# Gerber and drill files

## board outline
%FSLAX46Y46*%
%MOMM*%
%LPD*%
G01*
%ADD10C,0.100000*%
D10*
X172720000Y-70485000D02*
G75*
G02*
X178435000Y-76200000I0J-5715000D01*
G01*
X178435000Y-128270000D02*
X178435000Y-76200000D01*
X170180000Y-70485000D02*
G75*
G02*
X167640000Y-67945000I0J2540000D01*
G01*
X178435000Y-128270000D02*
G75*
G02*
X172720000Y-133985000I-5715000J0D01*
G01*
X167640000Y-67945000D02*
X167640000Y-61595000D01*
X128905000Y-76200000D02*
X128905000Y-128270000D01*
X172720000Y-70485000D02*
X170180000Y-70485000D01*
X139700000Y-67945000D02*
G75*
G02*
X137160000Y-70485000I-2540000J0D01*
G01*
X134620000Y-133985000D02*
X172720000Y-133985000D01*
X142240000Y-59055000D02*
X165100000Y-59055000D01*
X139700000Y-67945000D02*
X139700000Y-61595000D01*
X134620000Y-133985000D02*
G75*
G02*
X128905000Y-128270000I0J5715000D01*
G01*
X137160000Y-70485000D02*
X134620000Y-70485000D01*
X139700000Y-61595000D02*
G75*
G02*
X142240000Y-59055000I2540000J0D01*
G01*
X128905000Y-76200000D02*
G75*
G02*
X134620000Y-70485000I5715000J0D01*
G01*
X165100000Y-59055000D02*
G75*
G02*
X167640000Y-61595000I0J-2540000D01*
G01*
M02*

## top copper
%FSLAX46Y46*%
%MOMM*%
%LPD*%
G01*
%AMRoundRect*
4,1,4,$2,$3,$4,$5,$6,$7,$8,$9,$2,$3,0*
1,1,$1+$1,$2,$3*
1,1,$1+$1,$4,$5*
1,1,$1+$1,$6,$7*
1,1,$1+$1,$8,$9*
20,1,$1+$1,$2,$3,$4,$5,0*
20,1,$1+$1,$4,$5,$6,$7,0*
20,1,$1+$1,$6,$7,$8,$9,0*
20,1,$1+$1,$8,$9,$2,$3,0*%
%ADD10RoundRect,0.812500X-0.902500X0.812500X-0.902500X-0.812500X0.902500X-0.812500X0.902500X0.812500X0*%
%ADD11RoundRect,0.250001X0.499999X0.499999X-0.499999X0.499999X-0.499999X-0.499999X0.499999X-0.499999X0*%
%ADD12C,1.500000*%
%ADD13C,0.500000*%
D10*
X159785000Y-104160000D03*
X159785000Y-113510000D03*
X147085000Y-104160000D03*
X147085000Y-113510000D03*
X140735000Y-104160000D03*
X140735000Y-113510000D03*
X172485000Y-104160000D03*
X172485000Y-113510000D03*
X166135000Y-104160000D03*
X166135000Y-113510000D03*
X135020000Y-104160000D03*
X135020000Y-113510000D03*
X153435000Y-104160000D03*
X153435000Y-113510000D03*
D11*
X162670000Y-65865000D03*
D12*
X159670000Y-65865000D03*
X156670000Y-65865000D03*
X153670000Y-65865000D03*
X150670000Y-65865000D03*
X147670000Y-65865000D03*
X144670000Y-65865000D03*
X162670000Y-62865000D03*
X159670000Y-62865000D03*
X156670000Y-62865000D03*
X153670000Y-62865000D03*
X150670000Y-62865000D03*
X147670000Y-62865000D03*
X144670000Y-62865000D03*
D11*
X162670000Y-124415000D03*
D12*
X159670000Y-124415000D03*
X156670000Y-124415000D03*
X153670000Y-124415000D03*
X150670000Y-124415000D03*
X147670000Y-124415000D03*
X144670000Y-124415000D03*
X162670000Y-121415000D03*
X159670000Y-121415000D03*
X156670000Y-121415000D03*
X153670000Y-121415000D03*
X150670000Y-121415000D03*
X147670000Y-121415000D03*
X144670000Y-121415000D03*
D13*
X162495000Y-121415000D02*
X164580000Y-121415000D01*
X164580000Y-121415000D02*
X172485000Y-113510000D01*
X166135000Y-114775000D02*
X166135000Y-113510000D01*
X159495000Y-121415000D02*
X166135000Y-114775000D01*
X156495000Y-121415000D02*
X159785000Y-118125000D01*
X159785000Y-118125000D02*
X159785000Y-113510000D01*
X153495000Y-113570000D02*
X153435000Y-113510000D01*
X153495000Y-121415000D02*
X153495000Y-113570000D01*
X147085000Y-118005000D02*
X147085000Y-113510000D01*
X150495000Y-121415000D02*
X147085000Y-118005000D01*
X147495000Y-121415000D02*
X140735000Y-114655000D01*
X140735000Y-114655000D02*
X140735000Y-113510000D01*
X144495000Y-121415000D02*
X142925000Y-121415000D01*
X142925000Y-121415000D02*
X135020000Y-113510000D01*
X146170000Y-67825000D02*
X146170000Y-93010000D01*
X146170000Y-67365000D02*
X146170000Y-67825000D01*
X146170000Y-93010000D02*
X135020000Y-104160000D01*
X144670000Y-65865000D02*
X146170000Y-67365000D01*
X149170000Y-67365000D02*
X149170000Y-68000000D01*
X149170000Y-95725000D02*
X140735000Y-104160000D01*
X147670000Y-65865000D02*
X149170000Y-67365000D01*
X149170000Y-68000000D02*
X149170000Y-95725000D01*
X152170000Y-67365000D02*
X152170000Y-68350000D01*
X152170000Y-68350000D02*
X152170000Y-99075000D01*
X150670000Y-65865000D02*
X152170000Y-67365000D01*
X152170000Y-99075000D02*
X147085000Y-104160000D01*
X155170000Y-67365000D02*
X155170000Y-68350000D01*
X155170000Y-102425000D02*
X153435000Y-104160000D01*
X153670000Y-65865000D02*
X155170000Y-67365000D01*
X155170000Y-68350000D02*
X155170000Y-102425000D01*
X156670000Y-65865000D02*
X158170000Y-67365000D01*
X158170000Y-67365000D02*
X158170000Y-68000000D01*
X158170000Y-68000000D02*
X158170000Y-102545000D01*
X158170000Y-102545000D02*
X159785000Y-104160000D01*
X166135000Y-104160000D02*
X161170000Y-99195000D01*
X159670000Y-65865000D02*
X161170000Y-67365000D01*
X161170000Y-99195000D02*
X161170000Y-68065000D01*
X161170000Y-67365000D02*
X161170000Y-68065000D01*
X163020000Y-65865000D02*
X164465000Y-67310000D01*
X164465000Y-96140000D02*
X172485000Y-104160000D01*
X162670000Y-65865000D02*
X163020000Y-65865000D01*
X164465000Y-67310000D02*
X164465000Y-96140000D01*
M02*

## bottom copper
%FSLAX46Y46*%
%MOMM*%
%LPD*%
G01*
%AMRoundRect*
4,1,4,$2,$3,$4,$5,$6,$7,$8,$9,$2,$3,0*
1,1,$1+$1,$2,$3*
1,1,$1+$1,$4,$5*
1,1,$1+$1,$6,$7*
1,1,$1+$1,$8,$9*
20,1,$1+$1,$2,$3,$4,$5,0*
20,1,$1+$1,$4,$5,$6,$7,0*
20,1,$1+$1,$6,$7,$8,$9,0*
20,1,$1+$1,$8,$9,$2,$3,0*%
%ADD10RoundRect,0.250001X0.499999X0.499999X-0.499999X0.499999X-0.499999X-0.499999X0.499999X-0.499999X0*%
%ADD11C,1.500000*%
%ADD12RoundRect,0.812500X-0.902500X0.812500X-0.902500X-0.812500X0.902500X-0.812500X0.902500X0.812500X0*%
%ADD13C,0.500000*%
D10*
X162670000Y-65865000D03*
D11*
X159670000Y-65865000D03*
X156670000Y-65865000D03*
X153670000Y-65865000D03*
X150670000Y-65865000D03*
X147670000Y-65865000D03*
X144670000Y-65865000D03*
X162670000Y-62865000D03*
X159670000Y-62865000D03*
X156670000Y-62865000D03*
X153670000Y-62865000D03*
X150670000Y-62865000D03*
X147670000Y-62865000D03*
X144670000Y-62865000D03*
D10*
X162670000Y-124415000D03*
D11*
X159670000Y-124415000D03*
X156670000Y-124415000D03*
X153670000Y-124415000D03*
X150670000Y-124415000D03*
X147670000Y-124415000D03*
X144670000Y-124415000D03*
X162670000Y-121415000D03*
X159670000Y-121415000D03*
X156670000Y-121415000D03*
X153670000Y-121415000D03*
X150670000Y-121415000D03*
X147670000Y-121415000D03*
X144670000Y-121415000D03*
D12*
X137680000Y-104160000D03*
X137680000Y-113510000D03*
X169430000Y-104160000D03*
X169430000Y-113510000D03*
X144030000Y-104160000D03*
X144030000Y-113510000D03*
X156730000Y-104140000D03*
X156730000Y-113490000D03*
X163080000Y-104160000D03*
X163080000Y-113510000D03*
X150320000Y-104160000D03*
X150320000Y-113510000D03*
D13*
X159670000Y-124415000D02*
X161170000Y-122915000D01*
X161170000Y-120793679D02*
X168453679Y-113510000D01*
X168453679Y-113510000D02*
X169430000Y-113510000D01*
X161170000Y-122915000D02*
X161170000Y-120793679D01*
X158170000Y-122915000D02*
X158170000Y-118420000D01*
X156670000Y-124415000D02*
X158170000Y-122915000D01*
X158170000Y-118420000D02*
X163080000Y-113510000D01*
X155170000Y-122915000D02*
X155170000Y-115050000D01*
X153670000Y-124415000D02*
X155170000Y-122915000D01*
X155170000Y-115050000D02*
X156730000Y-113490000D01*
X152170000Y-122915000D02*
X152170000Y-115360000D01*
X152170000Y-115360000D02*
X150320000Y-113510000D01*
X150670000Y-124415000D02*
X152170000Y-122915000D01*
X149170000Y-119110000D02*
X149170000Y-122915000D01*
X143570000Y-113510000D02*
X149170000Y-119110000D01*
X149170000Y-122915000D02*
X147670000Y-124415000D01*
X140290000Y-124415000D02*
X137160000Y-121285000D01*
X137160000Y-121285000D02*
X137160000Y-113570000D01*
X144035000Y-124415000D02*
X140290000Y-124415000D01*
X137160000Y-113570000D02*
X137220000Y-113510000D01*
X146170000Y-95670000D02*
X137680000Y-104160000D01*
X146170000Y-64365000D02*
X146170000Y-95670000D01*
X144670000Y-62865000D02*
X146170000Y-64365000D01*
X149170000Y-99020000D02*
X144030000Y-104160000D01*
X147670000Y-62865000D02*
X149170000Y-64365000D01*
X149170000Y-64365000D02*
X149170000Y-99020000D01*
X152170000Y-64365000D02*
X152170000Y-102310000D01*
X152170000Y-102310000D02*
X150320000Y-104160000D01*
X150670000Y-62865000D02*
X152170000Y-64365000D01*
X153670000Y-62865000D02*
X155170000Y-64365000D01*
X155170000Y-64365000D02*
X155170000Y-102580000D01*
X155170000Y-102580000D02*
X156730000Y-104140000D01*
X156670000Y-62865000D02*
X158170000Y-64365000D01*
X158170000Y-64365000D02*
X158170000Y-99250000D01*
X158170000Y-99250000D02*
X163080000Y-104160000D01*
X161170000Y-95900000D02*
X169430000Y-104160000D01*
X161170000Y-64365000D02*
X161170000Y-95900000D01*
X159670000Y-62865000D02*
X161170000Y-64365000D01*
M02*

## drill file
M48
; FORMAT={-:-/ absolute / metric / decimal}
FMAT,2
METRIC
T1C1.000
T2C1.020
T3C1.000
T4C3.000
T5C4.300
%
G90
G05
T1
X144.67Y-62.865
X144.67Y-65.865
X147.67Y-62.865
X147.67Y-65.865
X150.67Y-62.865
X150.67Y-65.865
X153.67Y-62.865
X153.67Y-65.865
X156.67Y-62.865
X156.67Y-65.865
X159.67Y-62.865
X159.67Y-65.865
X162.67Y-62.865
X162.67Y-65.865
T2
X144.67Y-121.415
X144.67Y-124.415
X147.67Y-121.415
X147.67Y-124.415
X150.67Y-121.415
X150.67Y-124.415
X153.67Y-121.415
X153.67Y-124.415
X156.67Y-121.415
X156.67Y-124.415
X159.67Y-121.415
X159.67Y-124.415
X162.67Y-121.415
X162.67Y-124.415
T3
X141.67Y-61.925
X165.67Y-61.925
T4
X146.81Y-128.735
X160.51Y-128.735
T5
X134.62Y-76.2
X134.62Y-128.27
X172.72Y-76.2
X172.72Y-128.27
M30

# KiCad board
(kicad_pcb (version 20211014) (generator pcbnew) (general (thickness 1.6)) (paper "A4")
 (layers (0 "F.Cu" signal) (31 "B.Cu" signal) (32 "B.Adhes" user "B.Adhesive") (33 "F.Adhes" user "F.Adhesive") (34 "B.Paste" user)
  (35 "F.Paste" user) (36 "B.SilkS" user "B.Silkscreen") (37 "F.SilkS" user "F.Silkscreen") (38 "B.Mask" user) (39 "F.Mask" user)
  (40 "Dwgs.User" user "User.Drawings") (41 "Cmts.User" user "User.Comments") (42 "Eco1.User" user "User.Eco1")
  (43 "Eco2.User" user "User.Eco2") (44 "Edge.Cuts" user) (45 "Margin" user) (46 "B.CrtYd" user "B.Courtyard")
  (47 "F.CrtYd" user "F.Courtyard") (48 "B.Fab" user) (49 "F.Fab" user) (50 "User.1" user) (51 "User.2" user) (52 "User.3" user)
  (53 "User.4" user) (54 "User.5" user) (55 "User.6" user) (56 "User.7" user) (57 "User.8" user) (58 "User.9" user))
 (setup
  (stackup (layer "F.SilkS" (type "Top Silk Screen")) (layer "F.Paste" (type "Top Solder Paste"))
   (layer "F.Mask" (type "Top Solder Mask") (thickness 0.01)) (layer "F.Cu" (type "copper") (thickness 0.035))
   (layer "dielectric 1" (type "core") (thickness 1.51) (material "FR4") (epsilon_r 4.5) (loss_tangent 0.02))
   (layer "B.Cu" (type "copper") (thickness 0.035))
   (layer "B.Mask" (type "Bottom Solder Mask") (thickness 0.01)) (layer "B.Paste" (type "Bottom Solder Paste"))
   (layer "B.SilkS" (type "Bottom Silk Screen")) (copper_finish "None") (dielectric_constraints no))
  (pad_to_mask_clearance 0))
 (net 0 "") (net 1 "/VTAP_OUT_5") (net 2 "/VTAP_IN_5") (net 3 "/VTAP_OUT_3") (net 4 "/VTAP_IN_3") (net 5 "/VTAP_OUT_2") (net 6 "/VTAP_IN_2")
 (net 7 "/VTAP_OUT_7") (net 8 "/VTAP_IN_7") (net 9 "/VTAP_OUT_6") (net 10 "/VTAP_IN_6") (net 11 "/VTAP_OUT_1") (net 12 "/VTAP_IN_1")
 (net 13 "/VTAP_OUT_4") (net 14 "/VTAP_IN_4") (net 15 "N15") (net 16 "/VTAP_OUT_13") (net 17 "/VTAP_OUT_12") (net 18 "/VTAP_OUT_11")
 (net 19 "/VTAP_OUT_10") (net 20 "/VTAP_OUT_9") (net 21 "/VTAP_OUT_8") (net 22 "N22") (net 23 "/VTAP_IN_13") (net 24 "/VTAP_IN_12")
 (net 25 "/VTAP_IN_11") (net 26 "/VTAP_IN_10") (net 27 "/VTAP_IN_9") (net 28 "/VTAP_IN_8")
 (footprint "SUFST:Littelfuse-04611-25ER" (layer "F.Cu") (at 159.845 108.585 -90)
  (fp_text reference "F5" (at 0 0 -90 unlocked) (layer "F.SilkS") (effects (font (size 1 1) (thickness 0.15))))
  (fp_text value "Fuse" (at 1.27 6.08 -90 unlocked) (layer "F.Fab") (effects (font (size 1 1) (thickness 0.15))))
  (pad "1" smd roundrect (at -4.425 0.06 270) (size 3.25 3.43) (layers "F.Cu" "F.Paste" "F.Mask") (roundrect_rratio 0.25)
   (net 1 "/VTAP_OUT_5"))
  (pad "2" smd roundrect (at 4.925 0.06 270) (size 3.25 3.43) (layers "F.Cu" "F.Paste" "F.Mask") (roundrect_rratio 0.25)
   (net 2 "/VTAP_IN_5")))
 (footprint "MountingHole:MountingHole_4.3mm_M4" (layer "F.Cu") (at 172.72 76.2)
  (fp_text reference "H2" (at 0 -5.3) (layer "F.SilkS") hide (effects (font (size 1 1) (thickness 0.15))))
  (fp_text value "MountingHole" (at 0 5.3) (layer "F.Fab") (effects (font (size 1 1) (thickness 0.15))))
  (pad "" np_thru_hole circle (at 0 0) (size 4.3 4.3) (drill 4.3) (layers *.Cu *.Mask)))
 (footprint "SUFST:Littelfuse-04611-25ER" (layer "F.Cu") (at 147.145 108.585 -90)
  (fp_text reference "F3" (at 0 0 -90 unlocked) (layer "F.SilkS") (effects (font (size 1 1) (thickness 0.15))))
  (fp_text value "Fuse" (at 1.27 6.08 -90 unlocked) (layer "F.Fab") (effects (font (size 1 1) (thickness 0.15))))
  (pad "1" smd roundrect (at -4.425 0.06 270) (size 3.25 3.43) (layers "F.Cu" "F.Paste" "F.Mask") (roundrect_rratio 0.25)
   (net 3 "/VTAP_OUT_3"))
  (pad "2" smd roundrect (at 4.925 0.06 270) (size 3.25 3.43) (layers "F.Cu" "F.Paste" "F.Mask") (roundrect_rratio 0.25)
   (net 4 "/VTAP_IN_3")))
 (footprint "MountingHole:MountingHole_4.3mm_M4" (layer "F.Cu") (at 172.72 128.27)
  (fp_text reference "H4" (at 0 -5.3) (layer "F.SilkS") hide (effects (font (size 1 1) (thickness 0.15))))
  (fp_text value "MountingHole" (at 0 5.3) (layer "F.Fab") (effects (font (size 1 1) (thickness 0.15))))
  (pad "" np_thru_hole circle (at 0 0) (size 4.3 4.3) (drill 4.3) (layers *.Cu *.Mask)))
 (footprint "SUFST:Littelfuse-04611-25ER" (layer "F.Cu") (at 140.795 108.585 -90)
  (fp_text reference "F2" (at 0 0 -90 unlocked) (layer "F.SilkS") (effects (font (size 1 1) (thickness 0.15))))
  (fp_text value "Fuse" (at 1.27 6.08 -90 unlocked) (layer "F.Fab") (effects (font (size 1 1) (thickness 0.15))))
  (pad "1" smd roundrect (at -4.425 0.06 270) (size 3.25 3.43) (layers "F.Cu" "F.Paste" "F.Mask") (roundrect_rratio 0.25)
   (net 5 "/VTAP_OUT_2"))
  (pad "2" smd roundrect (at 4.925 0.06 270) (size 3.25 3.43) (layers "F.Cu" "F.Paste" "F.Mask") (roundrect_rratio 0.25)
   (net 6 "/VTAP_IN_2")))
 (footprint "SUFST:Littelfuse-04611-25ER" (layer "F.Cu") (at 172.545 108.585 -90)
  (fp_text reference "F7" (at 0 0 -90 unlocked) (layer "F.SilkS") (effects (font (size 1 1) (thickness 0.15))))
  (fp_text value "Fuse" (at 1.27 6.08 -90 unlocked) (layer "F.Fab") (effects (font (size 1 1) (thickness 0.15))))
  (pad "1" smd roundrect (at -4.425 0.06 270) (size 3.25 3.43) (layers "F.Cu" "F.Paste" "F.Mask") (roundrect_rratio 0.25)
   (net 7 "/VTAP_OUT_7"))
  (pad "2" smd roundrect (at 4.925 0.06 270) (size 3.25 3.43) (layers "F.Cu" "F.Paste" "F.Mask") (roundrect_rratio 0.25)
   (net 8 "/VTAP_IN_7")))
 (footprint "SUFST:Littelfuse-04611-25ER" (layer "F.Cu") (at 166.195 108.585 -90)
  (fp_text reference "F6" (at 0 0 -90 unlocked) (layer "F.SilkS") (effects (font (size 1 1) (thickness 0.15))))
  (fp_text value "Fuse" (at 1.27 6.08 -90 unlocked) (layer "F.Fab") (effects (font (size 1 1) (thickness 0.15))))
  (pad "1" smd roundrect (at -4.425 0.06 270) (size 3.25 3.43) (layers "F.Cu" "F.Paste" "F.Mask") (roundrect_rratio 0.25)
   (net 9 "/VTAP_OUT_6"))
  (pad "2" smd roundrect (at 4.925 0.06 270) (size 3.25 3.43) (layers "F.Cu" "F.Paste" "F.Mask") (roundrect_rratio 0.25)
   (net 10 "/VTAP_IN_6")))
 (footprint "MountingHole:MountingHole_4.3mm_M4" (layer "F.Cu") (at 134.62 128.27)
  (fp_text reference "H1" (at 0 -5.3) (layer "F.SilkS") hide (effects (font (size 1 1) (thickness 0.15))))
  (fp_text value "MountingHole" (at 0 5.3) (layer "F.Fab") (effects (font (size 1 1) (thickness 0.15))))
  (pad "" np_thru_hole circle (at 0 0) (size 4.3 4.3) (drill 4.3) (layers *.Cu *.Mask)))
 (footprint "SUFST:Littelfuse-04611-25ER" (layer "F.Cu") (at 135.08 108.585 -90)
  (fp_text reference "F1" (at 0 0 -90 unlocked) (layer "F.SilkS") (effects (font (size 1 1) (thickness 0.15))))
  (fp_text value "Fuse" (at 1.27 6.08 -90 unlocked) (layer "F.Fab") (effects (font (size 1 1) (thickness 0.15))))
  (pad "1" smd roundrect (at -4.425 0.06 270) (size 3.25 3.43) (layers "F.Cu" "F.Paste" "F.Mask") (roundrect_rratio 0.25)
   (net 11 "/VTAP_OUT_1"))
  (pad "2" smd roundrect (at 4.925 0.06 270) (size 3.25 3.43) (layers "F.Cu" "F.Paste" "F.Mask") (roundrect_rratio 0.25)
   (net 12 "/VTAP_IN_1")))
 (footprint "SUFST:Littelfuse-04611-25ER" (layer "F.Cu") (at 153.495 108.585 -90)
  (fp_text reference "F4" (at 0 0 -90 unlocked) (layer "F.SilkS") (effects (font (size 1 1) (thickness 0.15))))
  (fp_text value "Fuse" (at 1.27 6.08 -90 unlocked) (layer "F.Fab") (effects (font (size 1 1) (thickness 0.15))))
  (pad "1" smd roundrect (at -4.425 0.06 270) (size 3.25 3.43) (layers "F.Cu" "F.Paste" "F.Mask") (roundrect_rratio 0.25)
   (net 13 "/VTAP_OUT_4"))
  (pad "2" smd roundrect (at 4.925 0.06 270) (size 3.25 3.43) (layers "F.Cu" "F.Paste" "F.Mask") (roundrect_rratio 0.25)
   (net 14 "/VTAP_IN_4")))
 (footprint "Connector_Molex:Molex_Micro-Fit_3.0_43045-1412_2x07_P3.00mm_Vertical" (layer "F.Cu") (at 162.67 65.865 180)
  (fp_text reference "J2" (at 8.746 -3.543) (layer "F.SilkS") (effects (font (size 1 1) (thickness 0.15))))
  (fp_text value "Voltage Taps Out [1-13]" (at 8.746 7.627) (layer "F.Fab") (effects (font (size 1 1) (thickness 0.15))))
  (pad "" np_thru_hole circle (at 21 3.94 180) (size 1 1) (drill 1) (layers *.Cu *.Mask))
  (pad "" np_thru_hole circle (at -3 3.94 180) (size 1 1) (drill 1) (layers *.Cu *.Mask))
  (pad "1" thru_hole roundrect (at 0 0 180) (size 1.5 1.5) (drill 1) (layers *.Cu *.Mask) (roundrect_rratio 0.166667) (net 7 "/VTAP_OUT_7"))
  (pad "2" thru_hole circle (at 3 0 180) (size 1.5 1.5) (drill 1) (layers *.Cu *.Mask) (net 9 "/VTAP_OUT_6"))
  (pad "3" thru_hole circle (at 6 0 180) (size 1.5 1.5) (drill 1) (layers *.Cu *.Mask) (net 1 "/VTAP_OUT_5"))
  (pad "4" thru_hole circle (at 9 0 180) (size 1.5 1.5) (drill 1) (layers *.Cu *.Mask) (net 13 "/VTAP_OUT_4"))
  (pad "5" thru_hole circle (at 12 0 180) (size 1.5 1.5) (drill 1) (layers *.Cu *.Mask) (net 3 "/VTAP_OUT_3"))
  (pad "6" thru_hole circle (at 15 0 180) (size 1.5 1.5) (drill 1) (layers *.Cu *.Mask) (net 5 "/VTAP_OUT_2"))
  (pad "7" thru_hole circle (at 18 0 180) (size 1.5 1.5) (drill 1) (layers *.Cu *.Mask) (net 11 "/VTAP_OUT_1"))
  (pad "8" thru_hole circle (at 0 3 180) (size 1.5 1.5) (drill 1) (layers *.Cu *.Mask) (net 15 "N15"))
  (pad "9" thru_hole circle (at 3 3 180) (size 1.5 1.5) (drill 1) (layers *.Cu *.Mask) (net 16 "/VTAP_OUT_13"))
  (pad "10" thru_hole circle (at 6 3 180) (size 1.5 1.5) (drill 1) (layers *.Cu *.Mask) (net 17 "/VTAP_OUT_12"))
  (pad "11" thru_hole circle (at 9 3 180) (size 1.5 1.5) (drill 1) (layers *.Cu *.Mask) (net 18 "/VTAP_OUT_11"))
  (pad "12" thru_hole circle (at 12 3 180) (size 1.5 1.5) (drill 1) (layers *.Cu *.Mask) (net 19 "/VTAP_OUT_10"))
  (pad "13" thru_hole circle (at 15 3 180) (size 1.5 1.5) (drill 1) (layers *.Cu *.Mask) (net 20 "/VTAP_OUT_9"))
  (pad "14" thru_hole circle (at 18 3 180) (size 1.5 1.5) (drill 1) (layers *.Cu *.Mask) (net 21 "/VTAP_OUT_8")))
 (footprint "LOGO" (layer "F.Cu") (at 153.67 85.09)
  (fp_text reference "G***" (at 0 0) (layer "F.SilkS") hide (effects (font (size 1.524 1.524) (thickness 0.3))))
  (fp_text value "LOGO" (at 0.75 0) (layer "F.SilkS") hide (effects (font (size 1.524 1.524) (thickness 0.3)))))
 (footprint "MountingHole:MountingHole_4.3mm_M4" (layer "F.Cu") (at 134.62 76.2)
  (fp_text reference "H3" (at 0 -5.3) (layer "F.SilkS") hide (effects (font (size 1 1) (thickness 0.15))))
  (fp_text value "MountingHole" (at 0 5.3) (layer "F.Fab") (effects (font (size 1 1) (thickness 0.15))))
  (pad "" np_thru_hole circle (at 0 0) (size 4.3 4.3) (drill 4.3) (layers *.Cu *.Mask)))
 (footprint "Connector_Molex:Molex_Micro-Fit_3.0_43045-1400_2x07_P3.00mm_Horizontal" (layer "F.Cu") (at 162.67 124.415 180)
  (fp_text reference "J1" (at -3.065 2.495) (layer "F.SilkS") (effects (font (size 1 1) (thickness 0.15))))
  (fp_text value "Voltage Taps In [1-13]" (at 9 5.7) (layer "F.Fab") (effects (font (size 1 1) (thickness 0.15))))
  (pad "" np_thru_hole circle (at 15.86 -4.32 180) (size 3 3) (drill 3) (layers *.Cu *.Mask))
  (pad "" np_thru_hole circle (at 2.16 -4.32 180) (size 3 3) (drill 3) (layers *.Cu *.Mask))
  (pad "1" thru_hole roundrect (at 0 0 180) (size 1.5 1.5) (drill 1.02) (layers *.Cu *.Mask) (roundrect_rratio 0.166667) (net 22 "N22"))
  (pad "2" thru_hole circle (at 3 0 180) (size 1.5 1.5) (drill 1.02) (layers *.Cu *.Mask) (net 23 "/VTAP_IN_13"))
  (pad "3" thru_hole circle (at 6 0 180) (size 1.5 1.5) (drill 1.02) (layers *.Cu *.Mask) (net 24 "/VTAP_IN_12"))
  (pad "4" thru_hole circle (at 9 0 180) (size 1.5 1.5) (drill 1.02) (layers *.Cu *.Mask) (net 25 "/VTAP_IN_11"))
  (pad "5" thru_hole circle (at 12 0 180) (size 1.5 1.5) (drill 1.02) (layers *.Cu *.Mask) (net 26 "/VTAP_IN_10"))
  (pad "6" thru_hole circle (at 15 0 180) (size 1.5 1.5) (drill 1.02) (layers *.Cu *.Mask) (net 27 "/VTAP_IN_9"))
  (pad "7" thru_hole circle (at 18 0 180) (size 1.5 1.5) (drill 1.02) (layers *.Cu *.Mask) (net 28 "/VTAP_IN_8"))
  (pad "8" thru_hole circle (at 0 3 180) (size 1.5 1.5) (drill 1.02) (layers *.Cu *.Mask) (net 8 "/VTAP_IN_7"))
  (pad "9" thru_hole circle (at 3 3 180) (size 1.5 1.5) (drill 1.02) (layers *.Cu *.Mask) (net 10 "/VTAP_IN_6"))
  (pad "10" thru_hole circle (at 6 3 180) (size 1.5 1.5) (drill 1.02) (layers *.Cu *.Mask) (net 2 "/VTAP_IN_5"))
  (pad "11" thru_hole circle (at 9 3 180) (size 1.5 1.5) (drill 1.02) (layers *.Cu *.Mask) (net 14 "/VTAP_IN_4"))
  (pad "12" thru_hole circle (at 12 3 180) (size 1.5 1.5) (drill 1.02) (layers *.Cu *.Mask) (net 4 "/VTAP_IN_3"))
  (pad "13" thru_hole circle (at 15 3 180) (size 1.5 1.5) (drill 1.02) (layers *.Cu *.Mask) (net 6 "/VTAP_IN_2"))
  (pad "14" thru_hole circle (at 18 3 180) (size 1.5 1.5) (drill 1.02) (layers *.Cu *.Mask) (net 12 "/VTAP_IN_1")))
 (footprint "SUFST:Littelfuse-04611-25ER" (layer "B.Cu") (at 137.62 108.585 -90)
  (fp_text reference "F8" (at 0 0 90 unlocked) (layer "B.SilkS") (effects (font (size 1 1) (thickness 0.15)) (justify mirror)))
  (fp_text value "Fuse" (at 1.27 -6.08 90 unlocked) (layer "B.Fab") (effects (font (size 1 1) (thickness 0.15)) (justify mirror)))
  (pad "1" smd roundrect (at -4.425 -0.06 270) (size 3.25 3.43) (layers "B.Cu" "B.Paste" "B.Mask") (roundrect_rratio 0.25)
   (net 21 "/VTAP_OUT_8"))
  (pad "2" smd roundrect (at 4.925 -0.06 270) (size 3.25 3.43) (layers "B.Cu" "B.Paste" "B.Mask") (roundrect_rratio 0.25)
   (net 28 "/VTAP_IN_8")))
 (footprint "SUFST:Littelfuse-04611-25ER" (layer "B.Cu") (at 169.37 108.585 -90)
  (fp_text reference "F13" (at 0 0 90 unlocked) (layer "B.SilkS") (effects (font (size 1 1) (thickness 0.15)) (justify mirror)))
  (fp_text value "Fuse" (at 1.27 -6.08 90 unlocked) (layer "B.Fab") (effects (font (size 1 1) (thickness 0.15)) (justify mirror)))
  (pad "1" smd roundrect (at -4.425 -0.06 270) (size 3.25 3.43) (layers "B.Cu" "B.Paste" "B.Mask") (roundrect_rratio 0.25)
   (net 16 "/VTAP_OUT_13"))
  (pad "2" smd roundrect (at 4.925 -0.06 270) (size 3.25 3.43) (layers "B.Cu" "B.Paste" "B.Mask") (roundrect_rratio 0.25)
   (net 23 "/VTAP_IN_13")))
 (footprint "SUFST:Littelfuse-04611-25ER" (layer "B.Cu") (at 143.97 108.585 -90)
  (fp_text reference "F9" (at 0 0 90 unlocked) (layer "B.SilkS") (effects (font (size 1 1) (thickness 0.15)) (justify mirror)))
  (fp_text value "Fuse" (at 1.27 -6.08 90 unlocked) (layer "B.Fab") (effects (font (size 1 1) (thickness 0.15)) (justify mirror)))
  (pad "1" smd roundrect (at -4.425 -0.06 270) (size 3.25 3.43) (layers "B.Cu" "B.Paste" "B.Mask") (roundrect_rratio 0.25)
   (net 20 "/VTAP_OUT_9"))
  (pad "2" smd roundrect (at 4.925 -0.06 270) (size 3.25 3.43) (layers "B.Cu" "B.Paste" "B.Mask") (roundrect_rratio 0.25)
   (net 27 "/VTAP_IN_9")))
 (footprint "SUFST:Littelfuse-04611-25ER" (layer "B.Cu") (at 156.67 108.565 -90)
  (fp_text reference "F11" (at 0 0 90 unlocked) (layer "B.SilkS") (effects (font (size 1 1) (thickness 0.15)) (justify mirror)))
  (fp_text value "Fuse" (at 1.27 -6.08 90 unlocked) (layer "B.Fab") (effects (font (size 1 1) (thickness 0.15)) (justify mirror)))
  (pad "1" smd roundrect (at -4.425 -0.06 270) (size 3.25 3.43) (layers "B.Cu" "B.Paste" "B.Mask") (roundrect_rratio 0.25)
   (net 18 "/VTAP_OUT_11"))
  (pad "2" smd roundrect (at 4.925 -0.06 270) (size 3.25 3.43) (layers "B.Cu" "B.Paste" "B.Mask") (roundrect_rratio 0.25)
   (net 25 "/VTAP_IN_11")))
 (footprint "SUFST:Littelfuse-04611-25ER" (layer "B.Cu") (at 163.02 108.585 -90)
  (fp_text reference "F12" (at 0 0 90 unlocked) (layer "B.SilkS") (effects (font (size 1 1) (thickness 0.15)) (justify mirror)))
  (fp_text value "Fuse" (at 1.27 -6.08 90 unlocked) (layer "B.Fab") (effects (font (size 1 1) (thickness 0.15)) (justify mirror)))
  (pad "1" smd roundrect (at -4.425 -0.06 270) (size 3.25 3.43) (layers "B.Cu" "B.Paste" "B.Mask") (roundrect_rratio 0.25)
   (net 17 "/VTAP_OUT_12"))
  (pad "2" smd roundrect (at 4.925 -0.06 270) (size 3.25 3.43) (layers "B.Cu" "B.Paste" "B.Mask") (roundrect_rratio 0.25)
   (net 24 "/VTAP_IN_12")))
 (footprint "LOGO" (layer "B.Cu") (at 153.67 85.09 180)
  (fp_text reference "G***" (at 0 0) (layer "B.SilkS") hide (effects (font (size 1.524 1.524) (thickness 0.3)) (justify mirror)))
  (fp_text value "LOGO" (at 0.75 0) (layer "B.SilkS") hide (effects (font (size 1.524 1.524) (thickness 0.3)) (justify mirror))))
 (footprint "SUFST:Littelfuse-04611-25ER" (layer "B.Cu") (at 150.26 108.585 -90)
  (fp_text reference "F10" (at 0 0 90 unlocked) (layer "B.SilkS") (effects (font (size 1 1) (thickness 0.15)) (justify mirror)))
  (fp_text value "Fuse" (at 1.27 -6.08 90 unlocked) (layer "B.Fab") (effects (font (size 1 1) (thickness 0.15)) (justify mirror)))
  (pad "1" smd roundrect (at -4.425 -0.06 270) (size 3.25 3.43) (layers "B.Cu" "B.Paste" "B.Mask") (roundrect_rratio 0.25)
   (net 19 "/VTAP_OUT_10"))
  (pad "2" smd roundrect (at 4.925 -0.06 270) (size 3.25 3.43) (layers "B.Cu" "B.Paste" "B.Mask") (roundrect_rratio 0.25)
   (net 26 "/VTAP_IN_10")))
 (gr_arc (start 172.72 70.485) (mid 176.761115 72.158885) (end 178.435 76.2) (layer "Edge.Cuts") (width 0.1))
 (gr_line (start 178.435 128.27) (end 178.435 76.2) (layer "Edge.Cuts") (width 0.1))
 (gr_arc (start 170.18 70.485) (mid 168.383949 69.741051) (end 167.64 67.945) (layer "Edge.Cuts") (width 0.1))
 (gr_arc (start 178.435 128.27) (mid 176.761115 132.311115) (end 172.72 133.985) (layer "Edge.Cuts") (width 0.1))
 (gr_line (start 167.64 67.945) (end 167.64 61.595) (layer "Edge.Cuts") (width 0.1))
 (gr_line (start 128.905 76.2) (end 128.905 128.27) (layer "Edge.Cuts") (width 0.1))
 (gr_line (start 172.72 70.485) (end 170.18 70.485) (layer "Edge.Cuts") (width 0.1))
 (gr_arc (start 139.7 67.945) (mid 138.956051 69.741051) (end 137.16 70.485) (layer "Edge.Cuts") (width 0.1))
 (gr_line (start 134.62 133.985) (end 172.72 133.985) (layer "Edge.Cuts") (width 0.1))
 (gr_line (start 142.24 59.055) (end 165.1 59.055) (layer "Edge.Cuts") (width 0.1))
 (gr_line (start 139.7 67.945) (end 139.7 61.595) (layer "Edge.Cuts") (width 0.1))
 (gr_arc (start 134.62 133.985) (mid 130.578885 132.311115) (end 128.905 128.27) (layer "Edge.Cuts") (width 0.1))
 (gr_line (start 137.16 70.485) (end 134.62 70.485) (layer "Edge.Cuts") (width 0.1))
 (gr_arc (start 139.7 61.595) (mid 140.443949 59.798949) (end 142.24 59.055) (layer "Edge.Cuts") (width 0.1))
 (gr_arc (start 128.905 76.2) (mid 130.578885 72.158885) (end 134.62 70.485) (layer "Edge.Cuts") (width 0.1))
 (gr_arc (start 165.1 59.055) (mid 166.896051 59.798949) (end 167.64 61.595) (layer "Edge.Cuts") (width 0.1))
 (segment (start 159.67 124.415) (end 161.17 122.915) (width 0.5) (layer "B.Cu") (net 23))
 (segment (start 161.17 120.793679) (end 168.453679 113.51) (width 0.5) (layer "B.Cu") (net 23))
 (segment (start 168.453679 113.51) (end 169.43 113.51) (width 0.5) (layer "B.Cu") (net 23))
 (segment (start 161.17 122.915) (end 161.17 120.793679) (width 0.5) (layer "B.Cu") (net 23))
 (segment (start 158.17 122.915) (end 158.17 118.42) (width 0.5) (layer "B.Cu") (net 24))
 (segment (start 156.67 124.415) (end 158.17 122.915) (width 0.5) (layer "B.Cu") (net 24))
 (segment (start 158.17 118.42) (end 163.08 113.51) (width 0.5) (layer "B.Cu") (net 24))
 (segment (start 155.17 122.915) (end 155.17 115.05) (width 0.5) (layer "B.Cu") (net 25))
 (segment (start 153.67 124.415) (end 155.17 122.915) (width 0.5) (layer "B.Cu") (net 25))
 (segment (start 155.17 115.05) (end 156.73 113.49) (width 0.5) (layer "B.Cu") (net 25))
 (segment (start 152.17 122.915) (end 152.17 115.36) (width 0.5) (layer "B.Cu") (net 26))
 (segment (start 152.17 115.36) (end 150.32 113.51) (width 0.5) (layer "B.Cu") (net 26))
 (segment (start 150.67 124.415) (end 152.17 122.915) (width 0.5) (layer "B.Cu") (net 26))
 (segment (start 149.17 119.11) (end 149.17 122.915) (width 0.5) (layer "B.Cu") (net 27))
 (segment (start 143.57 113.51) (end 149.17 119.11) (width 0.5) (layer "B.Cu") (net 27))
 (segment (start 149.17 122.915) (end 147.67 124.415) (width 0.5) (layer "B.Cu") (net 27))
 (segment (start 140.29 124.415) (end 137.16 121.285) (width 0.5) (layer "B.Cu") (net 28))
 (segment (start 137.16 121.285) (end 137.16 113.57) (width 0.5) (layer "B.Cu") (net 28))
 (segment (start 144.035 124.415) (end 140.29 124.415) (width 0.5) (layer "B.Cu") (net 28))
 (segment (start 137.16 113.57) (end 137.22 113.51) (width 0.5) (layer "B.Cu") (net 28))
 (segment (start 162.495 121.415) (end 164.58 121.415) (width 0.5) (layer "F.Cu") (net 8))
 (segment (start 164.58 121.415) (end 172.485 113.51) (width 0.5) (layer "F.Cu") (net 8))
 (segment (start 166.135 114.775) (end 166.135 113.51) (width 0.5) (layer "F.Cu") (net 10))
 (segment (start 159.495 121.415) (end 166.135 114.775) (width 0.5) (layer "F.Cu") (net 10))
 (segment (start 156.495 121.415) (end 159.785 118.125) (width 0.5) (layer "F.Cu") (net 2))
 (segment (start 159.785 118.125) (end 159.785 113.51) (width 0.5) (layer "F.Cu") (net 2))
 (segment (start 153.495 113.57) (end 153.435 113.51) (width 0.5) (layer "F.Cu") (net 14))
 (segment (start 153.495 121.415) (end 153.495 113.57) (width 0.5) (layer "F.Cu") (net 14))
 (segment (start 147.085 118.005) (end 147.085 113.51) (width 0.5) (layer "F.Cu") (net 4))
 (segment (start 150.495 121.415) (end 147.085 118.005) (width 0.5) (layer "F.Cu") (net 4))
 (segment (start 147.495 121.415) (end 140.735 114.655) (width 0.5) (layer "F.Cu") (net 6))
 (segment (start 140.735 114.655) (end 140.735 113.51) (width 0.5) (layer "F.Cu") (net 6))
 (segment (start 144.495 121.415) (end 142.925 121.415) (width 0.5) (layer "F.Cu") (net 12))
 (segment (start 142.925 121.415) (end 135.02 113.51) (width 0.5) (layer "F.Cu") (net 12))
 (segment (start 146.17 67.825) (end 146.17 93.01) (width 0.5) (layer "F.Cu") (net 11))
 (segment (start 146.17 67.365) (end 146.17 67.825) (width 0.5) (layer "F.Cu") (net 11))
 (segment (start 146.17 93.01) (end 135.02 104.16) (width 0.5) (layer "F.Cu") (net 11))
 (segment (start 144.67 65.865) (end 146.17 67.365) (width 0.5) (layer "F.Cu") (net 11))
 (segment (start 149.17 67.365) (end 149.17 68) (width 0.5) (layer "F.Cu") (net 5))
 (segment (start 149.17 95.725) (end 140.735 104.16) (width 0.5) (layer "F.Cu") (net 5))
 (segment (start 147.67 65.865) (end 149.17 67.365) (width 0.5) (layer "F.Cu") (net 5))
 (segment (start 149.17 68) (end 149.17 95.725) (width 0.5) (layer "F.Cu") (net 5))
 (segment (start 152.17 67.365) (end 152.17 68.35) (width 0.5) (layer "F.Cu") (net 3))
 (segment (start 152.17 68.35) (end 152.17 99.075) (width 0.5) (layer "F.Cu") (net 3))
 (segment (start 150.67 65.865) (end 152.17 67.365) (width 0.5) (layer "F.Cu") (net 3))
 (segment (start 152.17 99.075) (end 147.085 104.16) (width 0.5) (layer "F.Cu") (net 3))
 (segment (start 155.17 67.365) (end 155.17 68.35) (width 0.5) (layer "F.Cu") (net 13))
 (segment (start 155.17 102.425) (end 153.435 104.16) (width 0.5) (layer "F.Cu") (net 13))
 (segment (start 153.67 65.865) (end 155.17 67.365) (width 0.5) (layer "F.Cu") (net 13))
 (segment (start 155.17 68.35) (end 155.17 102.425) (width 0.5) (layer "F.Cu") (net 13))
 (segment (start 156.67 65.865) (end 158.17 67.365) (width 0.5) (layer "F.Cu") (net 1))
 (segment (start 158.17 67.365) (end 158.17 68) (width 0.5) (layer "F.Cu") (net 1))
 (segment (start 158.17 68) (end 158.17 102.545) (width 0.5) (layer "F.Cu") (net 1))
 (segment (start 158.17 102.545) (end 159.785 104.16) (width 0.5) (layer "F.Cu") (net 1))
 (segment (start 166.135 104.16) (end 161.17 99.195) (width 0.5) (layer "F.Cu") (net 9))
 (segment (start 159.67 65.865) (end 161.17 67.365) (width 0.5) (layer "F.Cu") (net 9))
 (segment (start 161.17 99.195) (end 161.17 68.065) (width 0.5) (layer "F.Cu") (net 9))
 (segment (start 161.17 67.365) (end 161.17 68.065) (width 0.5) (layer "F.Cu") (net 9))
 (segment (start 163.02 65.865) (end 164.465 67.31) (width 0.5) (layer "F.Cu") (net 7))
 (segment (start 164.465 96.14) (end 172.485 104.16) (width 0.5) (layer "F.Cu") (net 7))
 (segment (start 162.67 65.865) (end 163.02 65.865) (width 0.5) (layer "F.Cu") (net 7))
 (segment (start 164.465 67.31) (end 164.465 96.14) (width 0.5) (layer "F.Cu") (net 7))
 (segment (start 146.17 95.67) (end 137.68 104.16) (width 0.5) (layer "B.Cu") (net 21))
 (segment (start 146.17 64.365) (end 146.17 95.67) (width 0.5) (layer "B.Cu") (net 21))
 (segment (start 144.67 62.865) (end 146.17 64.365) (width 0.5) (layer "B.Cu") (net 21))
 (segment (start 149.17 99.02) (end 144.03 104.16) (width 0.5) (layer "B.Cu") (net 20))
 (segment (start 147.67 62.865) (end 149.17 64.365) (width 0.5) (layer "B.Cu") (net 20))
 (segment (start 149.17 64.365) (end 149.17 99.02) (width 0.5) (layer "B.Cu") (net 20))
 (segment (start 152.17 64.365) (end 152.17 102.31) (width 0.5) (layer "B.Cu") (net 19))
 (segment (start 152.17 102.31) (end 150.32 104.16) (width 0.5) (layer "B.Cu") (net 19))
 (segment (start 150.67 62.865) (end 152.17 64.365) (width 0.5) (layer "B.Cu") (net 19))
 (segment (start 153.67 62.865) (end 155.17 64.365) (width 0.5) (layer "B.Cu") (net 18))
 (segment (start 155.17 64.365) (end 155.17 102.58) (width 0.5) (layer "B.Cu") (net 18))
 (segment (start 155.17 102.58) (end 156.73 104.14) (width 0.5) (layer "B.Cu") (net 18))
 (segment (start 156.67 62.865) (end 158.17 64.365) (width 0.5) (layer "B.Cu") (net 17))
 (segment (start 158.17 64.365) (end 158.17 99.25) (width 0.5) (layer "B.Cu") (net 17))
 (segment (start 158.17 99.25) (end 163.08 104.16) (width 0.5) (layer "B.Cu") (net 17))
 (segment (start 161.17 95.9) (end 169.43 104.16) (width 0.5) (layer "B.Cu") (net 16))
 (segment (start 161.17 64.365) (end 161.17 95.9) (width 0.5) (layer "B.Cu") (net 16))
 (segment (start 159.67 62.865) (end 161.17 64.365) (width 0.5) (layer "B.Cu") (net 16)))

